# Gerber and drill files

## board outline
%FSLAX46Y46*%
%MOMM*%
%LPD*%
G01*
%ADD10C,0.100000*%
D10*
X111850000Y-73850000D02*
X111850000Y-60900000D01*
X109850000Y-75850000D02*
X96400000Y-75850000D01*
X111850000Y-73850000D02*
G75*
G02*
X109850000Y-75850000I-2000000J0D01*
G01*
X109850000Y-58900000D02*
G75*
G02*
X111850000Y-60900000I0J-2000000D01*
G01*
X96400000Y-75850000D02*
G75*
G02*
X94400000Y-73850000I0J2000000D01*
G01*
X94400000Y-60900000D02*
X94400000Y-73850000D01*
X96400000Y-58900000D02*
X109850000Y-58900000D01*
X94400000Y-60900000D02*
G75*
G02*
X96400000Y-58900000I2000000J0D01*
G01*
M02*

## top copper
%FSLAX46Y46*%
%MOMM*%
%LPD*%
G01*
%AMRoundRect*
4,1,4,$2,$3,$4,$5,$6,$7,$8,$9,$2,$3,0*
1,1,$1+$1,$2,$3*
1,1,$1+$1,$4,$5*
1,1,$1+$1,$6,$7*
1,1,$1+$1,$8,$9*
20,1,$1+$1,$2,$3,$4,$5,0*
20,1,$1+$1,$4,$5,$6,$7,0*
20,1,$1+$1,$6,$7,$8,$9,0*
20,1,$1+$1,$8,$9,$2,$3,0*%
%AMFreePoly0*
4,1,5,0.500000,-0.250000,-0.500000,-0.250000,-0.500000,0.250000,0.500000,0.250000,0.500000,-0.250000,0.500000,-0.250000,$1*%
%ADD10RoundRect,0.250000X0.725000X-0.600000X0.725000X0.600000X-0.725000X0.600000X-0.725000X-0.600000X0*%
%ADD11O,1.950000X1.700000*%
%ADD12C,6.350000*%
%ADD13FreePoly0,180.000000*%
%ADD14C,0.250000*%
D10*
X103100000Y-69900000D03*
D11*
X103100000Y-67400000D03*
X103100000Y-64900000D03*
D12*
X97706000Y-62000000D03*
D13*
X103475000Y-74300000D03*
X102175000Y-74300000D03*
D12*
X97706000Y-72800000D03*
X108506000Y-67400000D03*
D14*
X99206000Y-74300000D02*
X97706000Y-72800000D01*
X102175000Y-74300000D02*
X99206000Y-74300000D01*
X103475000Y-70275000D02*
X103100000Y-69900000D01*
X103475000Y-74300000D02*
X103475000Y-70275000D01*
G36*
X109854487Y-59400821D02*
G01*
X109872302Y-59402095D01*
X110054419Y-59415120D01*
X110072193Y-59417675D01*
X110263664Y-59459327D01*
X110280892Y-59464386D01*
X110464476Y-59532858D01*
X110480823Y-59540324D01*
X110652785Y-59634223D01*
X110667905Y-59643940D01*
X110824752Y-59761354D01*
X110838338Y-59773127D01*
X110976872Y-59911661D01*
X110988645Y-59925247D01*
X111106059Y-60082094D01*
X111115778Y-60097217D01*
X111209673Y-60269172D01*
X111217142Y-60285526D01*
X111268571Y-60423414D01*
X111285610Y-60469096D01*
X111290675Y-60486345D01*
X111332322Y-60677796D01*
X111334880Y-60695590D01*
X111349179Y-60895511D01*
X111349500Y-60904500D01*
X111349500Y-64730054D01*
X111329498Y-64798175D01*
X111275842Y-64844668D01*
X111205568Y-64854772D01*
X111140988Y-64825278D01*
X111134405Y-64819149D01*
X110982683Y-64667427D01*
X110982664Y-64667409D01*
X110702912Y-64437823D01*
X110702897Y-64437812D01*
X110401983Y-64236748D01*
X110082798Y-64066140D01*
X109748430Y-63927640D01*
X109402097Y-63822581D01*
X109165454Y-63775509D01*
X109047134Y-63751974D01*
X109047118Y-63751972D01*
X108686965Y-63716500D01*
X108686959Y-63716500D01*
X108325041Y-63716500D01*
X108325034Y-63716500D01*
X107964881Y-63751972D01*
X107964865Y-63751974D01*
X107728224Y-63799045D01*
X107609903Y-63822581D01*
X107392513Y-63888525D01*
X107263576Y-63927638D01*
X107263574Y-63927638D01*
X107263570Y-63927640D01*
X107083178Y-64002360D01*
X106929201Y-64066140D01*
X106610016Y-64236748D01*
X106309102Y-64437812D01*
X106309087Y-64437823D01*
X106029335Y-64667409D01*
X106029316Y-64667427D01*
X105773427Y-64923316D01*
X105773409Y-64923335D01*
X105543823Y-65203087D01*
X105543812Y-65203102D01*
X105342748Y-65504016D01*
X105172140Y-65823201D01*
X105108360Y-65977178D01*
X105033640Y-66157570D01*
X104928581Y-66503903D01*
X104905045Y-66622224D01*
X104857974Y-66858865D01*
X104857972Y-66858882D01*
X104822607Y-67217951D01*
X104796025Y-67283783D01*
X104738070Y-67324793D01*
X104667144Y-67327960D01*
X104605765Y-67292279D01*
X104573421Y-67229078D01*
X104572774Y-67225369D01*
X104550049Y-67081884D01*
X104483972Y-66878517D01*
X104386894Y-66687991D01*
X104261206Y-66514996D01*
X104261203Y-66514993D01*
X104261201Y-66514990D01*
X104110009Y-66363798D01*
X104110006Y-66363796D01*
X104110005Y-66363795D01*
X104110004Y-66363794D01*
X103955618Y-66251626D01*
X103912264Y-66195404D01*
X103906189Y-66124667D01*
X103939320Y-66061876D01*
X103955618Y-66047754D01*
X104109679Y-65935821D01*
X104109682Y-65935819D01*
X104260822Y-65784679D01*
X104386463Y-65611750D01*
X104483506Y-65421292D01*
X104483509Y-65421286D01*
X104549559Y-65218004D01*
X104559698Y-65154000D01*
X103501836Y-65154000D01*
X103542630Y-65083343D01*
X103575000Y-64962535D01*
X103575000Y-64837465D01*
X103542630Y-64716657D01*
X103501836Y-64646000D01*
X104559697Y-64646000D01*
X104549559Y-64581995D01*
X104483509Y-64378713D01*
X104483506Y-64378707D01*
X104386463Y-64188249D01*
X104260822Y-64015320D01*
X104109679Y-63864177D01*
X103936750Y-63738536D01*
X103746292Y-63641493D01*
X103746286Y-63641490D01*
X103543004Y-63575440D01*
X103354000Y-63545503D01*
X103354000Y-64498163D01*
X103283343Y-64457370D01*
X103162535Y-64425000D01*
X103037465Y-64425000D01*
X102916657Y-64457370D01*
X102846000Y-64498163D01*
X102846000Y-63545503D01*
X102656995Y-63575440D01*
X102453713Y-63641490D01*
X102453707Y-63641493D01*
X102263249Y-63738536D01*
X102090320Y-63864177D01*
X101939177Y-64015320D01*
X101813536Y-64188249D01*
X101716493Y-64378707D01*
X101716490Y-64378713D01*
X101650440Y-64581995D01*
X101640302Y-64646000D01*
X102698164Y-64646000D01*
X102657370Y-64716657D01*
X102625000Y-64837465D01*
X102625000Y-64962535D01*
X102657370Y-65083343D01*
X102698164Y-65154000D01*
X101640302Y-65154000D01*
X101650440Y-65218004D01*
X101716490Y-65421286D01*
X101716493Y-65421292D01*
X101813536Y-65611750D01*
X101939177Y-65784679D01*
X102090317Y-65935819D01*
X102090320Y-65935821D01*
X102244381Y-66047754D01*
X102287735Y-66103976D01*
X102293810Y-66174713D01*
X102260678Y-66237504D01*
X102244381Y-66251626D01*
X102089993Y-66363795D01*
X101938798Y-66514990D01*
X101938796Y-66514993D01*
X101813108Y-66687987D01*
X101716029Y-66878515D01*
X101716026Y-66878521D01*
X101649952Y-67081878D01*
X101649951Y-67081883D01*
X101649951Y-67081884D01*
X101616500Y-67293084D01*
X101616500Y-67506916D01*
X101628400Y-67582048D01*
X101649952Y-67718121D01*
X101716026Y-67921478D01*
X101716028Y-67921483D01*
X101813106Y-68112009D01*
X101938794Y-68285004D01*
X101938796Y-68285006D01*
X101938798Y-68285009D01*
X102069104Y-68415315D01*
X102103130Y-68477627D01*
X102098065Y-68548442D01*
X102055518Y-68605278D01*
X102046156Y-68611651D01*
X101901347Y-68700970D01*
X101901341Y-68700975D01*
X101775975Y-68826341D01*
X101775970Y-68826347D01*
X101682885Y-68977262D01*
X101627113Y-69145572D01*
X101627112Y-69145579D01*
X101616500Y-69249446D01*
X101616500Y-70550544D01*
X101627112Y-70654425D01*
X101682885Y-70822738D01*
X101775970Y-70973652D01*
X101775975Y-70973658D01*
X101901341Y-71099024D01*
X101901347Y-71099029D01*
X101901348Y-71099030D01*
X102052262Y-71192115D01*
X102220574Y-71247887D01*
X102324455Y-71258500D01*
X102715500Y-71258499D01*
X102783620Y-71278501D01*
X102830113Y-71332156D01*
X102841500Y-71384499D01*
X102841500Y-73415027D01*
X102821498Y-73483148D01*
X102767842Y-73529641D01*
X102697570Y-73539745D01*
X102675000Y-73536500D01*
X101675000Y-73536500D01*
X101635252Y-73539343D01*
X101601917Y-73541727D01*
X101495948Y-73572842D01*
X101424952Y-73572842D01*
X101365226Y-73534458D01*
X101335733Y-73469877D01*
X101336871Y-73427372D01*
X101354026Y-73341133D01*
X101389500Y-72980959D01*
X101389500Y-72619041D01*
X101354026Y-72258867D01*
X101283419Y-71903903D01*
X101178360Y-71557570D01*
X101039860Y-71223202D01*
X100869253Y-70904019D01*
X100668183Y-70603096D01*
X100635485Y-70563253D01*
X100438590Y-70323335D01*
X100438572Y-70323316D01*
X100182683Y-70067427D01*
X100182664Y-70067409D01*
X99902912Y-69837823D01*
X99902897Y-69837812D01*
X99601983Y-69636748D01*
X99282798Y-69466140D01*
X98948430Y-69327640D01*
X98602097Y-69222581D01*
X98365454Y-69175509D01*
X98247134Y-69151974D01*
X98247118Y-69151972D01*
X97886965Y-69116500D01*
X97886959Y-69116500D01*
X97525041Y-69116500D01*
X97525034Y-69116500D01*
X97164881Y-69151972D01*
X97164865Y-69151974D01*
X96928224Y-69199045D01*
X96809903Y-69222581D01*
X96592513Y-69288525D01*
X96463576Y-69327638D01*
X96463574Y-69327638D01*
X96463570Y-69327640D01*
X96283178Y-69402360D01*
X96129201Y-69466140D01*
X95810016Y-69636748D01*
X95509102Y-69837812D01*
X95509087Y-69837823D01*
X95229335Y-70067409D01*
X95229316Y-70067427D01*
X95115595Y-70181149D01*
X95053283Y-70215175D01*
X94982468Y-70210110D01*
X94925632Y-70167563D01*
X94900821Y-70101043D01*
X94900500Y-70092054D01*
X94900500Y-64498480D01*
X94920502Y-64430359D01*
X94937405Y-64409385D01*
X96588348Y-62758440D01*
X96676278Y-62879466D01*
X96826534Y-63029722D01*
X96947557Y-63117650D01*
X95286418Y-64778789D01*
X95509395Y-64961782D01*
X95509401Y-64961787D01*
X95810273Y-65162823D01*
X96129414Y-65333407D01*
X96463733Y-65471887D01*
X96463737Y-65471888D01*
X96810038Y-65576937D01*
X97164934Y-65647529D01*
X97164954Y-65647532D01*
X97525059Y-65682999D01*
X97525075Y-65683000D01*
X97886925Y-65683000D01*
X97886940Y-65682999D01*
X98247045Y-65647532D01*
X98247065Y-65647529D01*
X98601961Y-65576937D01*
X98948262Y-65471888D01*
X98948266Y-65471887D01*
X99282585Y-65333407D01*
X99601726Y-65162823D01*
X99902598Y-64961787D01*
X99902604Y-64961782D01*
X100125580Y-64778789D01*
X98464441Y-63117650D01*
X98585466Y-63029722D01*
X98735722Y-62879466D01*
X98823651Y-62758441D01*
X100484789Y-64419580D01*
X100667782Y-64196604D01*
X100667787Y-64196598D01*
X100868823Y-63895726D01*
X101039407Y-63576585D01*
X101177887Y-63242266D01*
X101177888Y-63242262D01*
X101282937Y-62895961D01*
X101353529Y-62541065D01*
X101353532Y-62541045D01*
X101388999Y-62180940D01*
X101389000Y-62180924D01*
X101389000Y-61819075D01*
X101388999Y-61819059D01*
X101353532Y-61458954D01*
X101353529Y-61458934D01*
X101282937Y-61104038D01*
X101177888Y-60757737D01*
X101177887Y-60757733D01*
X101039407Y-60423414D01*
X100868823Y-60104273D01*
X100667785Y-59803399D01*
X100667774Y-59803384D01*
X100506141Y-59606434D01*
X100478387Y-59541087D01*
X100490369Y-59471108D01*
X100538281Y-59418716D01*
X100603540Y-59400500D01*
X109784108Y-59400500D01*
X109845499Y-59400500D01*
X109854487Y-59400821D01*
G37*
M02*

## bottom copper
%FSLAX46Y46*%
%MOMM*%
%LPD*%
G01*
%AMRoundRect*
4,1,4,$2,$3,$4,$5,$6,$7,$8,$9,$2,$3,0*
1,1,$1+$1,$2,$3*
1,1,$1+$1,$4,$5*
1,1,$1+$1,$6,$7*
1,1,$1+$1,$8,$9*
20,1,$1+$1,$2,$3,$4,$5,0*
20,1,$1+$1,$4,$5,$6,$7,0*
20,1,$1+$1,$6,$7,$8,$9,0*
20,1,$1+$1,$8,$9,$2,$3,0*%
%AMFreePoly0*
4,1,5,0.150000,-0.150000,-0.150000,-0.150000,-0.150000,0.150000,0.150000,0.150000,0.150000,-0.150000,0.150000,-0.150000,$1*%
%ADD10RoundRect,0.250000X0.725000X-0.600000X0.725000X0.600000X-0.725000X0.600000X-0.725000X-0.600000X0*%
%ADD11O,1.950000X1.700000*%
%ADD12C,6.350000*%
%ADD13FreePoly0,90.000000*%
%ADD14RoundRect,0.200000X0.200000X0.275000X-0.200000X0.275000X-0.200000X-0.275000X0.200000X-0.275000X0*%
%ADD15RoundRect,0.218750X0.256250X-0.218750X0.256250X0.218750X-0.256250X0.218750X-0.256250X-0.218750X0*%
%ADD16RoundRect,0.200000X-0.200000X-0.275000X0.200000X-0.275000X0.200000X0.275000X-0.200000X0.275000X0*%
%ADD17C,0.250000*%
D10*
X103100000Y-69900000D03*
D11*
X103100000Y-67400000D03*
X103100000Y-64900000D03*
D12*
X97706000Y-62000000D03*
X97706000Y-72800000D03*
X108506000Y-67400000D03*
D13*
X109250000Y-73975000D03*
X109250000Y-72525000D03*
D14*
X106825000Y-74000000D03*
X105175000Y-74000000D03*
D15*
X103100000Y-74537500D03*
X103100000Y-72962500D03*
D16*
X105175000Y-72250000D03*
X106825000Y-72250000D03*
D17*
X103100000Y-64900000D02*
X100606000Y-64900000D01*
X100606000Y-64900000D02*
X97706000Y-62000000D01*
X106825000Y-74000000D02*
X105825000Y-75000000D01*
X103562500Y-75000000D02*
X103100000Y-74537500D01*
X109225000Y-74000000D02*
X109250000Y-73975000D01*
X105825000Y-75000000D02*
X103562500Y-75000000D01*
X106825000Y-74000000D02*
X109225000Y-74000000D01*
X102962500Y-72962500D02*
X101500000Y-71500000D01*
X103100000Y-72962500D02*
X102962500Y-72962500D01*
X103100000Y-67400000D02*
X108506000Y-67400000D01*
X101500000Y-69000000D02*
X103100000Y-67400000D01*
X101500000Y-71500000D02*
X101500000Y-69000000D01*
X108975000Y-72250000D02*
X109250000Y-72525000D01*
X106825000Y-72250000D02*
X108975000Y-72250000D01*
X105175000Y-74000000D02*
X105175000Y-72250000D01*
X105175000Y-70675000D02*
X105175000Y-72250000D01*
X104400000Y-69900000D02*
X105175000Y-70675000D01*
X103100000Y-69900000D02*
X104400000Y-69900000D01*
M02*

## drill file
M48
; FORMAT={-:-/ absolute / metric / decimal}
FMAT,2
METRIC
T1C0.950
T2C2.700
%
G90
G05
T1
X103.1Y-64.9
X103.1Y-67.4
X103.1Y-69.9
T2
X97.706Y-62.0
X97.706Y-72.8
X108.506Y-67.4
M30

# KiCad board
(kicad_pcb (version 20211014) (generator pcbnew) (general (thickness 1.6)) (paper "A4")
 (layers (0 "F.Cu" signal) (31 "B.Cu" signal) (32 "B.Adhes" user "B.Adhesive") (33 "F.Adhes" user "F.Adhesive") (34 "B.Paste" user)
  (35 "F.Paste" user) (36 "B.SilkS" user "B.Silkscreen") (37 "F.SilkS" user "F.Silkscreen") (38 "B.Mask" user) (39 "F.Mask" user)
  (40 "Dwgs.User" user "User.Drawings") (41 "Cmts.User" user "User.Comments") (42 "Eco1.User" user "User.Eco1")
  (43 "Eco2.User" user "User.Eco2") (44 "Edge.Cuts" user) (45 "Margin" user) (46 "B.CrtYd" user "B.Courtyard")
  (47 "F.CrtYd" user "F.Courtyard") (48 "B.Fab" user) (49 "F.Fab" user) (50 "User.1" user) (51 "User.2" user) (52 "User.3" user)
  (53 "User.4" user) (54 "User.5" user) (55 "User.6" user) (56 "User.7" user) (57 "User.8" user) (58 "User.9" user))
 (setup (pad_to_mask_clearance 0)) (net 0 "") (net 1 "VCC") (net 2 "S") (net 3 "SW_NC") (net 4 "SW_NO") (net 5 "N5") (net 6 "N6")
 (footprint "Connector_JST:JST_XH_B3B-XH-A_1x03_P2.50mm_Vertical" (layer "F.Cu") (at 103.1 69.9 90)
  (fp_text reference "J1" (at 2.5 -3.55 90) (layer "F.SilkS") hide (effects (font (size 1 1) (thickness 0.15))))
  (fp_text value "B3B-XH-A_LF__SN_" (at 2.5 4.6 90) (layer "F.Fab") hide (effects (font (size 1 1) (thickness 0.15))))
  (pad "1" thru_hole roundrect locked (at 0 0 90) (size 1.7 1.95) (drill 0.95) (layers *.Cu *.Mask) (roundrect_rratio 0.1470588235)
   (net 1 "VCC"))
  (pad "2" thru_hole oval locked (at 2.5 0 90) (size 1.7 1.95) (drill 0.95) (layers *.Cu *.Mask) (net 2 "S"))
  (pad "3" thru_hole oval locked (at 5 0 90) (size 1.7 1.95) (drill 0.95) (layers *.Cu *.Mask) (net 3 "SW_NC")))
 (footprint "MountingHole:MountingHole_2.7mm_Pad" (layer "F.Cu") (at 97.706 62)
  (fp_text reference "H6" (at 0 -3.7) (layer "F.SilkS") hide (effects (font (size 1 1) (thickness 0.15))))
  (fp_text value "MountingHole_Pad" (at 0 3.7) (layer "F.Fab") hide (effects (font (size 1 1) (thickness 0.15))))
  (pad "1" thru_hole circle locked (at 0 0) (size 6.35 6.35) (drill 2.7) (layers *.Cu *.Mask) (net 3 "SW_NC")))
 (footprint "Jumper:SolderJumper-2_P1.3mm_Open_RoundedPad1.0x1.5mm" (layer "F.Cu") (at 102.825 74.3 180)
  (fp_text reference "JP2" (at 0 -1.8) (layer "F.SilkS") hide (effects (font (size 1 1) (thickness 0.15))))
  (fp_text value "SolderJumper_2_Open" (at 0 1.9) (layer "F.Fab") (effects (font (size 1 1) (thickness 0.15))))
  (pad "1" smd custom locked (at -0.65 0 180) (size 1 0.5) (layers "F.Cu" "F.Mask") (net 1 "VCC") (zone_connect 2)
   (options (clearance outline) (anchor rect)) (primitives))
  (pad "2" smd custom locked (at 0.65 0 180) (size 1 0.5) (layers "F.Cu" "F.Mask") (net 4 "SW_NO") (zone_connect 2)
   (options (clearance outline) (anchor rect)) (primitives)))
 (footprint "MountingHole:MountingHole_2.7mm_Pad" (layer "F.Cu") (at 97.706 72.8)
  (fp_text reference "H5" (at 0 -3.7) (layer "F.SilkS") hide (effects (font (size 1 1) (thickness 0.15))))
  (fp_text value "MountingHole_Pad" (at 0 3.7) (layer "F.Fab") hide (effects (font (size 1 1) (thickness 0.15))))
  (pad "1" thru_hole circle locked (at 0 0) (size 6.35 6.35) (drill 2.7) (layers *.Cu *.Mask) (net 4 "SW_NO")))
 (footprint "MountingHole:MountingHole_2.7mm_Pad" (layer "F.Cu") (at 108.506 67.4)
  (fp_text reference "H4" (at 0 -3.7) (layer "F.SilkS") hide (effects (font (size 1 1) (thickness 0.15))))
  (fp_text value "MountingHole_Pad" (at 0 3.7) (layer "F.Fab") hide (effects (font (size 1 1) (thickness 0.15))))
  (pad "1" thru_hole circle locked (at 0 0) (size 6.35 6.35) (drill 2.7) (layers *.Cu *.Mask) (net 2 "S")))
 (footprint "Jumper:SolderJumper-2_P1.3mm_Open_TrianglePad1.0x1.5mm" (layer "B.Cu") (at 109.25 73.25 90)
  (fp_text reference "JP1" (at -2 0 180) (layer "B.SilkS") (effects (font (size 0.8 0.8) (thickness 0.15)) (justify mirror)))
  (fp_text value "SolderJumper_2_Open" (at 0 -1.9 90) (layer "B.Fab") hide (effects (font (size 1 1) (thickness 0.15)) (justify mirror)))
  (pad "1" smd custom locked (at -0.725 0 90) (size 0.3 0.3) (layers "B.Cu" "B.Mask") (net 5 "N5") (zone_connect 2)
   (options (clearance outline) (anchor rect)) (primitives))
  (pad "2" smd custom locked (at 0.725 0 90) (size 0.3 0.3) (layers "B.Cu" "B.Mask") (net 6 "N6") (zone_connect 2)
   (options (clearance outline) (anchor rect)) (primitives)))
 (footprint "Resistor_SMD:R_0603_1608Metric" (layer "B.Cu") (at 106 74 180)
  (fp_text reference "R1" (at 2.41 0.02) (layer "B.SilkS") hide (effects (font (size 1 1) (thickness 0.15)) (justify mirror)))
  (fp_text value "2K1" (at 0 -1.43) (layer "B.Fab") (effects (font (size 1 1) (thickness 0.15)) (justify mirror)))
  (pad "1" smd roundrect locked (at -0.825 0 180) (size 0.8 0.95) (layers "B.Cu" "B.Paste" "B.Mask") (roundrect_rratio 0.25) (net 5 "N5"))
  (pad "2" smd roundrect locked (at 0.825 0 180) (size 0.8 0.95) (layers "B.Cu" "B.Paste" "B.Mask") (roundrect_rratio 0.25) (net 1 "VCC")))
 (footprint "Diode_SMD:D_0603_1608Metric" (layer "B.Cu") (at 103.1 73.75 90)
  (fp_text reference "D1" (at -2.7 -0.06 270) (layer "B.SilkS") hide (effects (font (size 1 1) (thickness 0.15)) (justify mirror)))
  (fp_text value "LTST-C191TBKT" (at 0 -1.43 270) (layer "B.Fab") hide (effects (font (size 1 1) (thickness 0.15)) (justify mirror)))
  (pad "1" smd roundrect (at -0.7875 0 90) (size 0.875 0.95) (layers "B.Cu" "B.Paste" "B.Mask") (roundrect_rratio 0.25) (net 5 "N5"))
  (pad "2" smd roundrect (at 0.7875 0 90) (size 0.875 0.95) (layers "B.Cu" "B.Paste" "B.Mask") (roundrect_rratio 0.25) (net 2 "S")))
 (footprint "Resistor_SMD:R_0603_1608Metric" (layer "B.Cu") (at 106 72.25)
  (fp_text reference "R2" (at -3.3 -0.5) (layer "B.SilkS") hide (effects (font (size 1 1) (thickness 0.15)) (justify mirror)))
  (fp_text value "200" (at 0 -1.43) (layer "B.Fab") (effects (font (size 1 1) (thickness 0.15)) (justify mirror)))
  (pad "1" smd roundrect locked (at -0.825 0) (size 0.8 0.95) (layers "B.Cu" "B.Paste" "B.Mask") (roundrect_rratio 0.25) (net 1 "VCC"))
  (pad "2" smd roundrect locked (at 0.825 0) (size 0.8 0.95) (layers "B.Cu" "B.Paste" "B.Mask") (roundrect_rratio 0.25) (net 6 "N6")))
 (gr_line (start 111.85 73.85) (end 111.85 60.9) (layer "Edge.Cuts") (width 0.1))
 (gr_line (start 109.85 75.85) (end 96.4 75.85) (layer "Edge.Cuts") (width 0.1))
 (gr_arc (start 111.85 73.85) (mid 111.264214 75.264214) (end 109.85 75.85) (layer "Edge.Cuts") (width 0.1))
 (gr_arc (start 109.85 58.9) (mid 111.264214 59.485786) (end 111.85 60.9) (layer "Edge.Cuts") (width 0.1))
 (gr_arc (start 96.4 75.85) (mid 94.985786 75.264214) (end 94.4 73.85) (layer "Edge.Cuts") (width 0.1))
 (gr_line (start 94.4 60.9) (end 94.4 73.85) (layer "Edge.Cuts") (width 0.1))
 (gr_line (start 96.4 58.9) (end 109.85 58.9) (layer "Edge.Cuts") (width 0.1))
 (gr_arc (start 94.4 60.9) (mid 94.985786 59.485786) (end 96.4 58.9) (layer "Edge.Cuts") (width 0.1))
 (segment (start 103.1 64.9) (end 100.606 64.9) (width 0.25) (layer "B.Cu") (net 3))
 (segment (start 100.606 64.9) (end 97.706 62) (width 0.25) (layer "B.Cu") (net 3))
 (segment (start 106.825 74) (end 105.825 75) (width 0.25) (layer "B.Cu") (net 5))
 (segment (start 103.5625 75) (end 103.1 74.5375) (width 0.25) (layer "B.Cu") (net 5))
 (segment (start 109.225 74) (end 109.25 73.975) (width 0.25) (layer "B.Cu") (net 5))
 (segment (start 105.825 75) (end 103.5625 75) (width 0.25) (layer "B.Cu") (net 5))
 (segment (start 106.825 74) (end 109.225 74) (width 0.25) (layer "B.Cu") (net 5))
 (segment (start 102.9625 72.9625) (end 101.5 71.5) (width 0.25) (layer "B.Cu") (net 2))
 (segment (start 103.1 72.9625) (end 102.9625 72.9625) (width 0.25) (layer "B.Cu") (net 2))
 (segment (start 103.1 67.4) (end 108.506 67.4) (width 0.25) (layer "B.Cu") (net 2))
 (segment (start 101.5 69) (end 103.1 67.4) (width 0.25) (layer "B.Cu") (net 2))
 (segment (start 101.5 71.5) (end 101.5 69) (width 0.25) (layer "B.Cu") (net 2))
 (segment (start 99.206 74.3) (end 97.706 72.8) (width 0.25) (layer "F.Cu") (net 4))
 (segment (start 102.175 74.3) (end 99.206 74.3) (width 0.25) (layer "F.Cu") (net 4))
 (segment (start 108.975 72.25) (end 109.25 72.525) (width 0.25) (layer "B.Cu") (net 6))
 (segment (start 106.825 72.25) (end 108.975 72.25) (width 0.25) (layer "B.Cu") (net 6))
 (segment (start 103.475 70.275) (end 103.1 69.9) (width 0.25) (layer "F.Cu") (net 1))
 (segment (start 103.475 74.3) (end 103.475 70.275) (width 0.25) (layer "F.Cu") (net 1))
 (segment (start 105.175 74) (end 105.175 72.25) (width 0.25) (layer "B.Cu") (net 1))
 (segment (start 105.175 70.675) (end 105.175 72.25) (width 0.25) (layer "B.Cu") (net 1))
 (segment (start 104.4 69.9) (end 105.175 70.675) (width 0.25) (layer "B.Cu") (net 1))
 (segment (start 103.1 69.9) (end 104.4 69.9) (width 0.25) (layer "B.Cu") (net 1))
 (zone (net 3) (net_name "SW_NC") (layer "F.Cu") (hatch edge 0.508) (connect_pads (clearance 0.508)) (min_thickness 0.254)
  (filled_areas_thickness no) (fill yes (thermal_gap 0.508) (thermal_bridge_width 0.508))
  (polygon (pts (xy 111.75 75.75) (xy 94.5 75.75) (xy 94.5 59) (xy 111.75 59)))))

